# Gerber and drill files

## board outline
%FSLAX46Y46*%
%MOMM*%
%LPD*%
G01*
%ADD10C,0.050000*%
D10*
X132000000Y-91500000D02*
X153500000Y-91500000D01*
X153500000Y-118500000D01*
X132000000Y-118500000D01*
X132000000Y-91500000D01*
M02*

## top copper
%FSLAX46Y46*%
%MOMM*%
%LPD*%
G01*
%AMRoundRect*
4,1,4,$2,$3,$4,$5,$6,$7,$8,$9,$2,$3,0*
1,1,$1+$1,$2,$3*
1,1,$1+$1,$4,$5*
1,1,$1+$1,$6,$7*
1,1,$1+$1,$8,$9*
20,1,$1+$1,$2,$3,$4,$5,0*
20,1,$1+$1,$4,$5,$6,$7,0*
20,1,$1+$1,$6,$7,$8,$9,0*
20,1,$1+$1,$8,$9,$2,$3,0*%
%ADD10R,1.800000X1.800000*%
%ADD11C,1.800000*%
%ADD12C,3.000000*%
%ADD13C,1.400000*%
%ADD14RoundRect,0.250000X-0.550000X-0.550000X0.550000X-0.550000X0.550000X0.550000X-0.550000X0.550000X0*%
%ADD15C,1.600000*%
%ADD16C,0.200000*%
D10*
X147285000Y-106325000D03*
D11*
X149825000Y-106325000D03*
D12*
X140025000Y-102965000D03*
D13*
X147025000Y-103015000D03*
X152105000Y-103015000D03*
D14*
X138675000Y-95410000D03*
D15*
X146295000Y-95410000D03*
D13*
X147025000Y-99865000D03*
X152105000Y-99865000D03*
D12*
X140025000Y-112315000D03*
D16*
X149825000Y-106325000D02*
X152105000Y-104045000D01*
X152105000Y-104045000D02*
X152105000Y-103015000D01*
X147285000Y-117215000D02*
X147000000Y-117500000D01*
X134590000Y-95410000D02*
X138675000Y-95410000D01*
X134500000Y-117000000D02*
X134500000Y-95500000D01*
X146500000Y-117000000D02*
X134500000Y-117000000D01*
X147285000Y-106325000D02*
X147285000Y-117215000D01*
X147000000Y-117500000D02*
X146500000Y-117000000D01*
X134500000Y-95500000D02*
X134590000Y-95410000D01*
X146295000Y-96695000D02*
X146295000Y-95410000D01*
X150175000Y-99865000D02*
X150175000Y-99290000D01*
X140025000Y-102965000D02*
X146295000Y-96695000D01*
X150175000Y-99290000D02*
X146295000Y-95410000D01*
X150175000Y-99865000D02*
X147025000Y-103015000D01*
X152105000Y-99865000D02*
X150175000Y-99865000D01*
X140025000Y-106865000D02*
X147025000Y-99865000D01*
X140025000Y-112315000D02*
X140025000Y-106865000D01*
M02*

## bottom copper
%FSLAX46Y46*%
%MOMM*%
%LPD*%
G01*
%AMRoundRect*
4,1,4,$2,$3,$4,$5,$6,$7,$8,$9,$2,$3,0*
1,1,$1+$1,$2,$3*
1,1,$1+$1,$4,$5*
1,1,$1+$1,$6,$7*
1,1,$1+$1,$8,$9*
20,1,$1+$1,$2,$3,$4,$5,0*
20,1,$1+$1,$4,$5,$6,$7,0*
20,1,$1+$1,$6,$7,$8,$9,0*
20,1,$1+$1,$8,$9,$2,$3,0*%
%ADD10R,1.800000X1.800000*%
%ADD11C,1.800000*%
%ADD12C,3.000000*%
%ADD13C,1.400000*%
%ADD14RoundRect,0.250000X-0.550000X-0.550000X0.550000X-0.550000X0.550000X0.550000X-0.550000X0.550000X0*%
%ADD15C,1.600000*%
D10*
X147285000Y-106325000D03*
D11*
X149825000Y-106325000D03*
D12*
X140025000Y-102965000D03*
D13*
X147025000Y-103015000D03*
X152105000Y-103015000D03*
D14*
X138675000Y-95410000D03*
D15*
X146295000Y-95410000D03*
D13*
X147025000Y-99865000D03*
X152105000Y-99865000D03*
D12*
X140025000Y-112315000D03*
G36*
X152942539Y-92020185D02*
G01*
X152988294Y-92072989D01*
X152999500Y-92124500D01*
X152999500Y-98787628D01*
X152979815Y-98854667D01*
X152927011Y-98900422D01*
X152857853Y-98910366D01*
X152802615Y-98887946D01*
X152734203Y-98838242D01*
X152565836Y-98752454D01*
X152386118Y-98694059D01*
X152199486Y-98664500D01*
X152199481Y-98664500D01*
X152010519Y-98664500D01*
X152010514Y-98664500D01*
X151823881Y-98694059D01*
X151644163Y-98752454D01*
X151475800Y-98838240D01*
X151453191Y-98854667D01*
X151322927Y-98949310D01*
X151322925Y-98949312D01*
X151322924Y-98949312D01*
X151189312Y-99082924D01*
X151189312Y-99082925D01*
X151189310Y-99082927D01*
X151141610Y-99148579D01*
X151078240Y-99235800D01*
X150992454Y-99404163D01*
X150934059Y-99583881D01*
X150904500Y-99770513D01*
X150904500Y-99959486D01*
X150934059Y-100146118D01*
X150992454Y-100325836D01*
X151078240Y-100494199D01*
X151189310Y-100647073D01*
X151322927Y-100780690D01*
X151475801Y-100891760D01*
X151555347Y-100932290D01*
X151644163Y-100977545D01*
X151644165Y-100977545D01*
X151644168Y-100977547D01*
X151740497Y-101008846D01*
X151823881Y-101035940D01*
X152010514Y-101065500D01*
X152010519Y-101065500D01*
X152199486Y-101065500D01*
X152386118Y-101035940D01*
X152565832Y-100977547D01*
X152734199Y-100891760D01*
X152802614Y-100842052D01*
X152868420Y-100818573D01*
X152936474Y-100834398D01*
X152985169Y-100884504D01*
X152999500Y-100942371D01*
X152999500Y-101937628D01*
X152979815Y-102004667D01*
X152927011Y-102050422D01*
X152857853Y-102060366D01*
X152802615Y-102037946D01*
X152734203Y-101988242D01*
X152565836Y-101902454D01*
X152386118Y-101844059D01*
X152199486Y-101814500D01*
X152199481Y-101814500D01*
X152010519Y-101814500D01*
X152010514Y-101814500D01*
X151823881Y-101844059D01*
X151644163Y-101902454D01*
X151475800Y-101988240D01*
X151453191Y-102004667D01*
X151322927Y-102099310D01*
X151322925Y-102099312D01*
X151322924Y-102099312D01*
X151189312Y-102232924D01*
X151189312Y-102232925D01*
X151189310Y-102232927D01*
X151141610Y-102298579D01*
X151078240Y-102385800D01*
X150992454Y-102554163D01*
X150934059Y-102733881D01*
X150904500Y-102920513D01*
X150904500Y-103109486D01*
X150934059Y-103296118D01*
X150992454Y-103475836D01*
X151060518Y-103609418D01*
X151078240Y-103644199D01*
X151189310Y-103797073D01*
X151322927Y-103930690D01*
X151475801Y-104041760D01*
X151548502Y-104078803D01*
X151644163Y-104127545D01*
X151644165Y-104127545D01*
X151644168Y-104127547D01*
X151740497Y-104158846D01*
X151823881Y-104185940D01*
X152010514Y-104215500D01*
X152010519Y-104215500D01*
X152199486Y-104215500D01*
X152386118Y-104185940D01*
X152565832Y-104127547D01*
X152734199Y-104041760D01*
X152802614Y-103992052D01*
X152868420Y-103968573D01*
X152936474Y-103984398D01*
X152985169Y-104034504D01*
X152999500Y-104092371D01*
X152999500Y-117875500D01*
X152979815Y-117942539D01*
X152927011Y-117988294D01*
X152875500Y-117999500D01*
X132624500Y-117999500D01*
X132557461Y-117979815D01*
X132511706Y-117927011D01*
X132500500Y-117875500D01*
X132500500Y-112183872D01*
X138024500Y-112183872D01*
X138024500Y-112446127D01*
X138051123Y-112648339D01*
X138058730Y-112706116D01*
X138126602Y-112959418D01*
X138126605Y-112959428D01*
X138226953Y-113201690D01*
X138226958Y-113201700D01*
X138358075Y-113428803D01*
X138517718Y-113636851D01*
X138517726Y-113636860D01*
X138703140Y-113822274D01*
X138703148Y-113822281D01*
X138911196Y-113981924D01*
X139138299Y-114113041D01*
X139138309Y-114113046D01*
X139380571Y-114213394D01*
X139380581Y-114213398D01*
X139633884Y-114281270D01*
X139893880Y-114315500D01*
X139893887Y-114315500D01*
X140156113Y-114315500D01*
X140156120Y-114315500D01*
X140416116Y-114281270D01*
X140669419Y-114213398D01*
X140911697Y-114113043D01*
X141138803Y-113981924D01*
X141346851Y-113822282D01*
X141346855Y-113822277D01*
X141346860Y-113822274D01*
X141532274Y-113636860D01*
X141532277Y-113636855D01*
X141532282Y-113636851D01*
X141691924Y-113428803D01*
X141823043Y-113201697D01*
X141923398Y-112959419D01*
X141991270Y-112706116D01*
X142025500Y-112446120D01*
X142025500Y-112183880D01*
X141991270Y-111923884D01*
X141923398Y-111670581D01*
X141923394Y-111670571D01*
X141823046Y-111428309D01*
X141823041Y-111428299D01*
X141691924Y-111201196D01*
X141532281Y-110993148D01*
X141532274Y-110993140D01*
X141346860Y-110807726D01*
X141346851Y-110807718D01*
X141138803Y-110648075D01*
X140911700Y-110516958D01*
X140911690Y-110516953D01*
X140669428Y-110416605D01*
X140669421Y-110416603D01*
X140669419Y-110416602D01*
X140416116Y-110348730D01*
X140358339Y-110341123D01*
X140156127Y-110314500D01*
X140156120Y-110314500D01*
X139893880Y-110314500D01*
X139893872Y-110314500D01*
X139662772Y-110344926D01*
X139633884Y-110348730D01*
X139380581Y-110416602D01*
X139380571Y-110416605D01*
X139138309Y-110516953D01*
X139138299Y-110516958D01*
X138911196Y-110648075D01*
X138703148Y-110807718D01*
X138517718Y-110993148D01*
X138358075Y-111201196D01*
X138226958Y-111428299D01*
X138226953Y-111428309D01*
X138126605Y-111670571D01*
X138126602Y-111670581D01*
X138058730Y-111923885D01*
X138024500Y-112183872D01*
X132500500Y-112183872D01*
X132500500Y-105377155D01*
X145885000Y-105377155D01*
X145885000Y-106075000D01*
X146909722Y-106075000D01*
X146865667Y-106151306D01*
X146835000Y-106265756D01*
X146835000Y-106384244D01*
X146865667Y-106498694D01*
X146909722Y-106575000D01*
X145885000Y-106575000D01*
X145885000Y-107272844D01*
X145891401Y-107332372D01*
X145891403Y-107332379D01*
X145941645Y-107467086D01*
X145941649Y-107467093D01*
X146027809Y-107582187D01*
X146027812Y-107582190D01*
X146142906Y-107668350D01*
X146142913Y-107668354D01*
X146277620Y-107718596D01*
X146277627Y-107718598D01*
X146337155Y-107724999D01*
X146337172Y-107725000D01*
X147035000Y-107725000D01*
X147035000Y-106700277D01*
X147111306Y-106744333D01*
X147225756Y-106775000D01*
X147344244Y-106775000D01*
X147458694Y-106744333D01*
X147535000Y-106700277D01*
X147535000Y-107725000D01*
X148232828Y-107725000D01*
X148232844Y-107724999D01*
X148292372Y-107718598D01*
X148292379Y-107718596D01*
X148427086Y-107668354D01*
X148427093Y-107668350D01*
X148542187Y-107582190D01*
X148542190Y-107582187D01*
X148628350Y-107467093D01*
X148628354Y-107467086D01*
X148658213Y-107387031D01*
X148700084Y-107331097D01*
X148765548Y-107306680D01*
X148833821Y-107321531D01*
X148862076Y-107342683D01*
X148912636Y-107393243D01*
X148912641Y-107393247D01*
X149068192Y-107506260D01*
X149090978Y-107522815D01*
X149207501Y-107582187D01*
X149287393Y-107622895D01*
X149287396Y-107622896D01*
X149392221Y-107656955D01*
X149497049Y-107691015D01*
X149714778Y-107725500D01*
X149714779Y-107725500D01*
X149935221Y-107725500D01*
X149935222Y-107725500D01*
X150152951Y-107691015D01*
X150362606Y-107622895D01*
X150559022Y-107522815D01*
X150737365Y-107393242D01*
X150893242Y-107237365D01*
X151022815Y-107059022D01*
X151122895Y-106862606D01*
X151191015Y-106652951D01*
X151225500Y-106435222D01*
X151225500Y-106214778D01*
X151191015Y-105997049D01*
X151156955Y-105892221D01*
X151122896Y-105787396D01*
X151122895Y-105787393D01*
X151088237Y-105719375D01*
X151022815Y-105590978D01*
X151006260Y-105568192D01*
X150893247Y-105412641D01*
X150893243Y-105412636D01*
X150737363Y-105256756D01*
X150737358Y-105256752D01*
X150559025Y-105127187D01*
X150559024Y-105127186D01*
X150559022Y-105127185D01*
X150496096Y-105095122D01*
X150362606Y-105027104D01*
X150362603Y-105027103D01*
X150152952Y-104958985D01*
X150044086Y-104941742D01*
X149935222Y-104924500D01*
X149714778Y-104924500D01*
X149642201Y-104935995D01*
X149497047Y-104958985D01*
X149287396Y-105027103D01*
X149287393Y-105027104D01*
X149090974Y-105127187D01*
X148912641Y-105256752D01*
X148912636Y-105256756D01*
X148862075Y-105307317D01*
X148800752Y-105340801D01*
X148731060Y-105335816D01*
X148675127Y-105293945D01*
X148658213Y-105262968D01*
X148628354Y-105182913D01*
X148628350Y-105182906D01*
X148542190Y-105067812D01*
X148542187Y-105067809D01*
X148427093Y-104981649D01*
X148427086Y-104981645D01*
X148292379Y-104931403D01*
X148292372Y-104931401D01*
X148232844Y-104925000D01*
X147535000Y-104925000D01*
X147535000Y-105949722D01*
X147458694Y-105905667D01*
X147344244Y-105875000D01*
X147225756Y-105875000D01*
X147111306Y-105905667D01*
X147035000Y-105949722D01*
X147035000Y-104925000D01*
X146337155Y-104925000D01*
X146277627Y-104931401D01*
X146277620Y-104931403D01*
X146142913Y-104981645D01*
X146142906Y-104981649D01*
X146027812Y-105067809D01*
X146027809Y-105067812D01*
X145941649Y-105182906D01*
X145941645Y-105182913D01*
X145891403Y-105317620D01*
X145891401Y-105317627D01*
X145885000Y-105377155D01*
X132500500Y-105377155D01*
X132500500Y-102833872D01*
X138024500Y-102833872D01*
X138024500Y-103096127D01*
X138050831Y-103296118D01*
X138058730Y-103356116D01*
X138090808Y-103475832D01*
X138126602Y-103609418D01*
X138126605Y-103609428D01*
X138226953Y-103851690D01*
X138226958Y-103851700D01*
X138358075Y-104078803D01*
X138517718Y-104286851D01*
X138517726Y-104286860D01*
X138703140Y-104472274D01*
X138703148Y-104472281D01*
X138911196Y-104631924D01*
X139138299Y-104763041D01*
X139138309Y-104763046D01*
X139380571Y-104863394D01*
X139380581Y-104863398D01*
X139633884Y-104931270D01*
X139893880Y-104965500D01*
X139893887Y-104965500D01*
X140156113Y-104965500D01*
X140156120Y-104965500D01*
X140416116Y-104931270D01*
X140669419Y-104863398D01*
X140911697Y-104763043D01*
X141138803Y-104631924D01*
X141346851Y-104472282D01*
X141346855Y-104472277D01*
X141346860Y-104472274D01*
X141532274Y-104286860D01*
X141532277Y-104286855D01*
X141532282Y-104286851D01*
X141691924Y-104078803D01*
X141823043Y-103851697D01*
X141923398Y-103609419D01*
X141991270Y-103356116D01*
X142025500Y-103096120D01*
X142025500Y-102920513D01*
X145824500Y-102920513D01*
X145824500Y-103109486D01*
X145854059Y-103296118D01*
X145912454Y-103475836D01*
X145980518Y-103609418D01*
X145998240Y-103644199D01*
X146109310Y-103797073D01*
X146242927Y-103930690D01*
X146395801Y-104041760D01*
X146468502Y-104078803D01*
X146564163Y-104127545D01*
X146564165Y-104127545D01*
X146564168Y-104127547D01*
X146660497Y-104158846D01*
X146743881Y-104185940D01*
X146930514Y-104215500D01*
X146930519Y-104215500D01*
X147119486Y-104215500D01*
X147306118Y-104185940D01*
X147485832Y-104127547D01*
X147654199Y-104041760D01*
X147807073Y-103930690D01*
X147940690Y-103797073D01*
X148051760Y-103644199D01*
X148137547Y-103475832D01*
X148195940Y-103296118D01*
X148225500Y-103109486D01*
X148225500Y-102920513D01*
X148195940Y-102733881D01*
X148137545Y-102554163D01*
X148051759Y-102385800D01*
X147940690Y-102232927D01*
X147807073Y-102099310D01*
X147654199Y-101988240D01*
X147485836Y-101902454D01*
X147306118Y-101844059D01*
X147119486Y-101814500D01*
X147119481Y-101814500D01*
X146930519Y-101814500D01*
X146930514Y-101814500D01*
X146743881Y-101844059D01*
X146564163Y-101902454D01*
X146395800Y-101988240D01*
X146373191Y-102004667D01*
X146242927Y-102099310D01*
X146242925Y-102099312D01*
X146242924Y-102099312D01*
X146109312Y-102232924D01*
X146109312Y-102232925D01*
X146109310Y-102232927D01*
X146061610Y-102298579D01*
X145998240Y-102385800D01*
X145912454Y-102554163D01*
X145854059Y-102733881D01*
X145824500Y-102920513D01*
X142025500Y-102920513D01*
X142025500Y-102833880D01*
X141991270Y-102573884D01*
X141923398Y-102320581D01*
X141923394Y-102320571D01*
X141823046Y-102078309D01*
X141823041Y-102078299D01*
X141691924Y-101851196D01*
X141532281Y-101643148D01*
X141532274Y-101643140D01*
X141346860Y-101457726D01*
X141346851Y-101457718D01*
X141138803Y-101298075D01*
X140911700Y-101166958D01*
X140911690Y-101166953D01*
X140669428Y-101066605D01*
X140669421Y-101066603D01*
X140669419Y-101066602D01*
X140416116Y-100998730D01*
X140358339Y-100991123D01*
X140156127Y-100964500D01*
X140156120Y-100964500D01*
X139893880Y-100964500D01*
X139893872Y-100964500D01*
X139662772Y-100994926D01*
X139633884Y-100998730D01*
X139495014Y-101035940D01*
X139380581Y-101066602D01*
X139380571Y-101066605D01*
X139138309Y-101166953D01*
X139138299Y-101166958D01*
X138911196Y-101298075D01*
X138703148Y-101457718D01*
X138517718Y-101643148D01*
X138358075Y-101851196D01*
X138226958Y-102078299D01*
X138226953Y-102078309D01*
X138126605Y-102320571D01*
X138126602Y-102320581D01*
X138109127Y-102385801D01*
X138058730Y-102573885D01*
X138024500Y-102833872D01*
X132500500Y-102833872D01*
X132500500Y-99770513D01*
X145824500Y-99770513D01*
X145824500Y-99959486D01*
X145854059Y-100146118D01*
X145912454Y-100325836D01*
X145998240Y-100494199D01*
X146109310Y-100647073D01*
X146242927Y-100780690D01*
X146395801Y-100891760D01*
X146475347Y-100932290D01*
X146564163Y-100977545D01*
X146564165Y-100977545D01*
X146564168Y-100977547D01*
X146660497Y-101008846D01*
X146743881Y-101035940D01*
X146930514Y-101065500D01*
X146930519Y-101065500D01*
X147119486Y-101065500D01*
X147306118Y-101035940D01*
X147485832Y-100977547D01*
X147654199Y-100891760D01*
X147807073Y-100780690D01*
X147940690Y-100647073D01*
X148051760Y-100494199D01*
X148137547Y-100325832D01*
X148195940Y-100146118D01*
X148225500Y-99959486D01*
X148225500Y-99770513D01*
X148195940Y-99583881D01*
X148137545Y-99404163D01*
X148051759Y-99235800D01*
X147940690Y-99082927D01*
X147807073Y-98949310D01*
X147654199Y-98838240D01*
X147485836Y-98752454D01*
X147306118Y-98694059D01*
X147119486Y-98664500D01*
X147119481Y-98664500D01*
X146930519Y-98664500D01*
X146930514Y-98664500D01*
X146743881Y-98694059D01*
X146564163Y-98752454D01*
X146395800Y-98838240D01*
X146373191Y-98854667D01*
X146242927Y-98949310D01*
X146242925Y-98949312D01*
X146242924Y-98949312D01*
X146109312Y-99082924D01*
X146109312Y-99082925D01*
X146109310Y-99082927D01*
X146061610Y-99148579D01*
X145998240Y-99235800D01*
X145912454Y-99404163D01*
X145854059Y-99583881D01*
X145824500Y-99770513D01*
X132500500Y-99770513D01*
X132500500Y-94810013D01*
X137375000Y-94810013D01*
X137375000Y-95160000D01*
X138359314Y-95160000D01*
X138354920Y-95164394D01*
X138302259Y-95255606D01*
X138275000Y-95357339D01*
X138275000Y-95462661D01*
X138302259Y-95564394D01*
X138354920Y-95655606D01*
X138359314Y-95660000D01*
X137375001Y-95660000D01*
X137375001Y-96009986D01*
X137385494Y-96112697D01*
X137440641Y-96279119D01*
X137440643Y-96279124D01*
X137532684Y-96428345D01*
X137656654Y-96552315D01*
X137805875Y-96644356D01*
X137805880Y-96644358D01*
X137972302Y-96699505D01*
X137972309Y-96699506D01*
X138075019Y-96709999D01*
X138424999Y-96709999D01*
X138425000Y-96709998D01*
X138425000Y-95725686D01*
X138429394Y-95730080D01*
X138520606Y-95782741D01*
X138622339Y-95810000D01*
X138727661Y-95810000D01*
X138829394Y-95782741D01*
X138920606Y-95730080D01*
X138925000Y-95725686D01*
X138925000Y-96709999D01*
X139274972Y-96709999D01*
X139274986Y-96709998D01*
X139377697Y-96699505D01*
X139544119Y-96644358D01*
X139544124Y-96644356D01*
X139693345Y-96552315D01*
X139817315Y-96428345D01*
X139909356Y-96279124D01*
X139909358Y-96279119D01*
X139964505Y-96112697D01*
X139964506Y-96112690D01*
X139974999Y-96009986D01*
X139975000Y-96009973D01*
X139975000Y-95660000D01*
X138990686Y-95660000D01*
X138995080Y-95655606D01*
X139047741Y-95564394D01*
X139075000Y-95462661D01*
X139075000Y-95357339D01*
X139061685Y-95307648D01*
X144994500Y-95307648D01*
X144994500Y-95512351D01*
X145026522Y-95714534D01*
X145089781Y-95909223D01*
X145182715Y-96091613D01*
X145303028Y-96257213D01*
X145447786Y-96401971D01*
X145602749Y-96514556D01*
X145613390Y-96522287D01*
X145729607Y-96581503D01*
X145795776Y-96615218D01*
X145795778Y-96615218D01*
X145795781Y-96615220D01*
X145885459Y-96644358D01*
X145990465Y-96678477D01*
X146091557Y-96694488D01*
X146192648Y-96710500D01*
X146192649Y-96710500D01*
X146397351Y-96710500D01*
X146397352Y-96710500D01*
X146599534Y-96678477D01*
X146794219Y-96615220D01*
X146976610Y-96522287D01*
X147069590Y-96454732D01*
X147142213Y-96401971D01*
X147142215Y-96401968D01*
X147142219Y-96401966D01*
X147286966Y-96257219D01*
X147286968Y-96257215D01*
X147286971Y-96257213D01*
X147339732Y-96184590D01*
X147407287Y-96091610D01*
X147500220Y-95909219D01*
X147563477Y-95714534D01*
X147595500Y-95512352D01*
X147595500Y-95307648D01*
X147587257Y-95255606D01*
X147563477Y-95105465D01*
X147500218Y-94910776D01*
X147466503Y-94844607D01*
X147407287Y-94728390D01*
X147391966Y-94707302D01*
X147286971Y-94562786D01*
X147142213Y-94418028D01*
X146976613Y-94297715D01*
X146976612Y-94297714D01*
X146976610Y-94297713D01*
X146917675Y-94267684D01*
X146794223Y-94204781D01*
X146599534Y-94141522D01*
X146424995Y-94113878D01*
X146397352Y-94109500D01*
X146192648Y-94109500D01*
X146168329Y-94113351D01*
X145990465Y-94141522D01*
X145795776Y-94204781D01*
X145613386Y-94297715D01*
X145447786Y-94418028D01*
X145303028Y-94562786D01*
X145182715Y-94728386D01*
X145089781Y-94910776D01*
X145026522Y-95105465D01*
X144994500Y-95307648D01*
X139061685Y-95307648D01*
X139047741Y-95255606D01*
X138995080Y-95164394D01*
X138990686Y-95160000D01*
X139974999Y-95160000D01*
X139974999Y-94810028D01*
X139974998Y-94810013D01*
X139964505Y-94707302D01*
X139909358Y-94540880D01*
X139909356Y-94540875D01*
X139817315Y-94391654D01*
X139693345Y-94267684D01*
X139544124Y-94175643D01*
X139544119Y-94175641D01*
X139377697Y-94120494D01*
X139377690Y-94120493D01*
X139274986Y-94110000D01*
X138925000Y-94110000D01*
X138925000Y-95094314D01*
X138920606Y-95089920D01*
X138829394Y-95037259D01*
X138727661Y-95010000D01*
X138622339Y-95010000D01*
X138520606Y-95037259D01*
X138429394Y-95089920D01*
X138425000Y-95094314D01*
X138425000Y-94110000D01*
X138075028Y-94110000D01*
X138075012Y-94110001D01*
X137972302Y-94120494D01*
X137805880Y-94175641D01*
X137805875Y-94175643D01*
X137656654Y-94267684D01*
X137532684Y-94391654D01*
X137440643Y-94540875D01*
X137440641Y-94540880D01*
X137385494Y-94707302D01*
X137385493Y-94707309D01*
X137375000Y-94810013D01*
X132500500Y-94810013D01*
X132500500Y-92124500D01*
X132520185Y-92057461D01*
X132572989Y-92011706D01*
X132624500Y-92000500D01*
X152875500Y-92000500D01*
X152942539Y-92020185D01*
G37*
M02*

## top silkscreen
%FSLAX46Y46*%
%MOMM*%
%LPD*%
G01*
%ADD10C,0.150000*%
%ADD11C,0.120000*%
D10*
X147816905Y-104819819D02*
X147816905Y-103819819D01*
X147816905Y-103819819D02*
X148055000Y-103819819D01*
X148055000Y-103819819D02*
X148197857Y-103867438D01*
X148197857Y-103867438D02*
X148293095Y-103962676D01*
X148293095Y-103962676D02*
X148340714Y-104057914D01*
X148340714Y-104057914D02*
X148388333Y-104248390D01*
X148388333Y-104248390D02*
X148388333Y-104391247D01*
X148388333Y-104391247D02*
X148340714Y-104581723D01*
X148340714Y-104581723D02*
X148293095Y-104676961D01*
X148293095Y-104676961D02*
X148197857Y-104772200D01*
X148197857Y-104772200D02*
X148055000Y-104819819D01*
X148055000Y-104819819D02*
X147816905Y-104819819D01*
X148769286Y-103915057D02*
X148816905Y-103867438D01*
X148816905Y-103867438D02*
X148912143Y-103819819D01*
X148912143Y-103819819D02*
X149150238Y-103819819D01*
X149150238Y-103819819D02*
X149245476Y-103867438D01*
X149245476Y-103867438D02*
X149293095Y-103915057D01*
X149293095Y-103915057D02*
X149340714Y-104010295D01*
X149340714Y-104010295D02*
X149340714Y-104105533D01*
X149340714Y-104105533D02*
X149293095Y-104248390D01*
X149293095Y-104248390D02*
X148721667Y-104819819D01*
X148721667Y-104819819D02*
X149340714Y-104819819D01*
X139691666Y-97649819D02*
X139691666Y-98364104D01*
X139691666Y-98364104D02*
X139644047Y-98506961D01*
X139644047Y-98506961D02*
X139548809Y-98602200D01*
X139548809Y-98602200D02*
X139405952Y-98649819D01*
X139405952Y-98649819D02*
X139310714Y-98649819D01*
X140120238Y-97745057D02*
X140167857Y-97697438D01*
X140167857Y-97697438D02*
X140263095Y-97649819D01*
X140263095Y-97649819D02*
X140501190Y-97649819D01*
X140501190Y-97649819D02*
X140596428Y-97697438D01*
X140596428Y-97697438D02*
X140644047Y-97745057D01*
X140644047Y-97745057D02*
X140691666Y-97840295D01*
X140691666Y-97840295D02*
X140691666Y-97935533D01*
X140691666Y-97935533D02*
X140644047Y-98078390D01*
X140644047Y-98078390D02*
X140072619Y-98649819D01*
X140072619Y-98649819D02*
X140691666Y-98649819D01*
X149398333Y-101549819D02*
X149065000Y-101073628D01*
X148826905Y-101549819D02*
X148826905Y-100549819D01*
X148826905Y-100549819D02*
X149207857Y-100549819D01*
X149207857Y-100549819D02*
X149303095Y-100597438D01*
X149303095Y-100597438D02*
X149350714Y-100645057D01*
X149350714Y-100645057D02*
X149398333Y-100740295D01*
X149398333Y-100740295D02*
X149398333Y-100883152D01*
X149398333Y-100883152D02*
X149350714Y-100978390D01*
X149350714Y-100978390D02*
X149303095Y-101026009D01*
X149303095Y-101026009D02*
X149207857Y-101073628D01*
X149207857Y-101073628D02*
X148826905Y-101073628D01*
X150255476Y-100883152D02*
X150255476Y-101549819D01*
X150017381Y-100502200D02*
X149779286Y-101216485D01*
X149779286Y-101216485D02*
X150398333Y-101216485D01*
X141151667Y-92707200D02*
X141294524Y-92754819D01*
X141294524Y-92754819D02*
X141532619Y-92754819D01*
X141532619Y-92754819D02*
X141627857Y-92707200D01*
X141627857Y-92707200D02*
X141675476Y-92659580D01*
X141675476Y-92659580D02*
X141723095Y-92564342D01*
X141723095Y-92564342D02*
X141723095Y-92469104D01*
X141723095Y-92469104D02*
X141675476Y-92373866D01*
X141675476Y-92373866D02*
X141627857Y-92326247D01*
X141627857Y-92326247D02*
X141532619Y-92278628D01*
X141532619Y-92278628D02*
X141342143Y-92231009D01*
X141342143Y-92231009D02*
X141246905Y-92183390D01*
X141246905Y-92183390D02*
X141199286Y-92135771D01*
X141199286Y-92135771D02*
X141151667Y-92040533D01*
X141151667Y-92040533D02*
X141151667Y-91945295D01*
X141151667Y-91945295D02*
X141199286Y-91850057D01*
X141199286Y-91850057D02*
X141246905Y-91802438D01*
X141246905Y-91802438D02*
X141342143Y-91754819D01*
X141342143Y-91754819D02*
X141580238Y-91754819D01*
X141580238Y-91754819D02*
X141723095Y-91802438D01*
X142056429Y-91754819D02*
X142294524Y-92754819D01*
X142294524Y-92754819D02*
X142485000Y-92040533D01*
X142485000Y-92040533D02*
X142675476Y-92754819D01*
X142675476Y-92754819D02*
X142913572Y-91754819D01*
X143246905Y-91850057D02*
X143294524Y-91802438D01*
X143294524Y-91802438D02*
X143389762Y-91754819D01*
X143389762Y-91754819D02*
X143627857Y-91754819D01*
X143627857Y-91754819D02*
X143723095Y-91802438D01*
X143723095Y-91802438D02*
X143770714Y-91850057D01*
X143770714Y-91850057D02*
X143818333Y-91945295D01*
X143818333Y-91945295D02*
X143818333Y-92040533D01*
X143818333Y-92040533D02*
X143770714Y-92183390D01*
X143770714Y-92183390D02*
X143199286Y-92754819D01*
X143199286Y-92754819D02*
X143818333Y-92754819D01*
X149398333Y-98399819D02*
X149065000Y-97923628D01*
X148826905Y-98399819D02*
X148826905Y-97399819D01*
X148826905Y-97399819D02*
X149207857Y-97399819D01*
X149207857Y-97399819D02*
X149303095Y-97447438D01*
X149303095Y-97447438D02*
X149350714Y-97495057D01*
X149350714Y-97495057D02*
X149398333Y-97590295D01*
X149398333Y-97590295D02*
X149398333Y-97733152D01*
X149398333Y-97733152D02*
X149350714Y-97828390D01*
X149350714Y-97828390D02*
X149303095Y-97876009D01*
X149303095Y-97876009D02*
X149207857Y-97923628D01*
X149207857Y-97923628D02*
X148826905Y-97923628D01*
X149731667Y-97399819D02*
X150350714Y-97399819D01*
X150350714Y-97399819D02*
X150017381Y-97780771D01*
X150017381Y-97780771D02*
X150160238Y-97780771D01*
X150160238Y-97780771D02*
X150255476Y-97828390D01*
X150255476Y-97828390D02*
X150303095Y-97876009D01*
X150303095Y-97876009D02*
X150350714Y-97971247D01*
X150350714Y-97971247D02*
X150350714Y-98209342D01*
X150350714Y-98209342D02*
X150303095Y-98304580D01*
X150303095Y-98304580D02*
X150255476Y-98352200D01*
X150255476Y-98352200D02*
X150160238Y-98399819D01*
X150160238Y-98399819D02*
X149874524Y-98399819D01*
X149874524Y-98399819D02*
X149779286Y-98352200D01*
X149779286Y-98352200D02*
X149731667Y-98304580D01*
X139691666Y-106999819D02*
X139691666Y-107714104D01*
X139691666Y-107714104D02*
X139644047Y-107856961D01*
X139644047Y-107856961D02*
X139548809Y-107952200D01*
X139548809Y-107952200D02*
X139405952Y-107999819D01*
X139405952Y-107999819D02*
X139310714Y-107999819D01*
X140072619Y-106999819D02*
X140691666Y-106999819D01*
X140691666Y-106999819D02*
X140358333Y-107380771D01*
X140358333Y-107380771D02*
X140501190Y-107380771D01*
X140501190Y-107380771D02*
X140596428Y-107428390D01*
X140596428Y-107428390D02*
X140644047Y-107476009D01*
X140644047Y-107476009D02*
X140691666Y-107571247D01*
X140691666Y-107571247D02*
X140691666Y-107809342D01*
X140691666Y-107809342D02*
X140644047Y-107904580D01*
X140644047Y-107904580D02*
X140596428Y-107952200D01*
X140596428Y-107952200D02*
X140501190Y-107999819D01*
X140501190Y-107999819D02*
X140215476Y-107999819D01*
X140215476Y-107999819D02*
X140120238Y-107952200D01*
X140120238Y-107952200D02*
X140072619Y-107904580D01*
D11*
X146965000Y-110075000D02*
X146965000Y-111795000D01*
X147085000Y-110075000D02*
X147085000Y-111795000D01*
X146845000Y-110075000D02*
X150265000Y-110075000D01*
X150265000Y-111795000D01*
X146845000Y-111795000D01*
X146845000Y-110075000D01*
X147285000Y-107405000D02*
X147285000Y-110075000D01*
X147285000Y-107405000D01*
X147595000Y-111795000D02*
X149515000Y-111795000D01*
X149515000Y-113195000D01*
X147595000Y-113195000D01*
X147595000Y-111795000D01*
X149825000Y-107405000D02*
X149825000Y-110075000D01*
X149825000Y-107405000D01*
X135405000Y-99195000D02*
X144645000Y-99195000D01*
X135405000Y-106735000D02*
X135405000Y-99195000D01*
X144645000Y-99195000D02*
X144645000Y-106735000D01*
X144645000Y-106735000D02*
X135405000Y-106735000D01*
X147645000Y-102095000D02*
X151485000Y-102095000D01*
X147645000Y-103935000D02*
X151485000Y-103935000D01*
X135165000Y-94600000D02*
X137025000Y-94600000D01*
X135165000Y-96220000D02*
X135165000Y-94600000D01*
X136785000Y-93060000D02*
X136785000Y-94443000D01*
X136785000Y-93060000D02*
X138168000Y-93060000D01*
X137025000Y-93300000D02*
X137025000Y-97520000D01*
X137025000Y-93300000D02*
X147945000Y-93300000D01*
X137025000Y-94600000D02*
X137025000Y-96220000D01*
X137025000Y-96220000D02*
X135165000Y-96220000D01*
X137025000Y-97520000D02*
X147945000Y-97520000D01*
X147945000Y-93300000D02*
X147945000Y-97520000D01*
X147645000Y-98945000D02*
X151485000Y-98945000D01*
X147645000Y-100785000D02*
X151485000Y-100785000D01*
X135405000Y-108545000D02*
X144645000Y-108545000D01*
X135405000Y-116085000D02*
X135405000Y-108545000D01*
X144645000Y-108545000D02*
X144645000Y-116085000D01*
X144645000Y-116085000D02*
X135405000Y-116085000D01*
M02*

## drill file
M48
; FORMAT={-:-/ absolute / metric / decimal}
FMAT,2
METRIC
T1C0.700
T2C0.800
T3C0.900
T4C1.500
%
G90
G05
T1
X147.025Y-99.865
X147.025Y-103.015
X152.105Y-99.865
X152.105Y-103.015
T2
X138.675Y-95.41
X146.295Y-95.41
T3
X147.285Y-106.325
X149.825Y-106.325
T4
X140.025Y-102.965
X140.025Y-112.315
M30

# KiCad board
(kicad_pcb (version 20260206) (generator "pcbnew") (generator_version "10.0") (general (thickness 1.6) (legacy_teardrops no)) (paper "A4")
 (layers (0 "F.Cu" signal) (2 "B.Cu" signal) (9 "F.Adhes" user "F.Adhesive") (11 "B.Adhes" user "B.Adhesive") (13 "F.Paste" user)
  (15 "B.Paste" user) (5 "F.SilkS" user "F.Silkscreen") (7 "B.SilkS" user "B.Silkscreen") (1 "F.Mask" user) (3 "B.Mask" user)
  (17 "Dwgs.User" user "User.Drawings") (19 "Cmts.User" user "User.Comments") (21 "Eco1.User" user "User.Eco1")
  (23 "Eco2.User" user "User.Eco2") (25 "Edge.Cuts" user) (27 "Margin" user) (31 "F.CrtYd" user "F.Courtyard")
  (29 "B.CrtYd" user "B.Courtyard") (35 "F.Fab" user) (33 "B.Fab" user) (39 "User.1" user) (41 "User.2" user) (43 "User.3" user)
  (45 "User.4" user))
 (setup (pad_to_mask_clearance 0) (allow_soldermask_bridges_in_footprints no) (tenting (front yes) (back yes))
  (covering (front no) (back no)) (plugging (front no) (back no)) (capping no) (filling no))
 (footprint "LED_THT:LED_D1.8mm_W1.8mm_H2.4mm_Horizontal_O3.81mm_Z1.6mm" (layer "F.Cu") (at 147.285 106.325)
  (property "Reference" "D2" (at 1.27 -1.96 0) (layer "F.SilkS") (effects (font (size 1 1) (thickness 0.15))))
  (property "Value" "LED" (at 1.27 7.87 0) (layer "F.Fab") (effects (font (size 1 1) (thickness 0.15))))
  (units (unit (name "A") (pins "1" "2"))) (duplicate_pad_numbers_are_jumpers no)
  (fp_line (start -0.32 3.75) (end -0.32 5.47) (stroke (width 0.12) (type solid)) (layer "F.SilkS"))
  (fp_line (start -0.2 3.75) (end -0.2 5.47) (stroke (width 0.12) (type solid)) (layer "F.SilkS"))
  (fp_rect (start -0.44 3.75) (end 2.98 5.47) (stroke (width 0.12) (type solid)) (fill no) (layer "F.SilkS"))
  (fp_rect (start 0 1.08) (end 0 3.75) (stroke (width 0.12) (type solid)) (fill no) (layer "F.SilkS"))
  (fp_rect (start 0.31 5.47) (end 2.23 6.87) (stroke (width 0.12) (type solid)) (fill no) (layer "F.SilkS"))
  (fp_rect (start 2.54 1.08) (end 2.54 3.75) (stroke (width 0.12) (type solid)) (fill no) (layer "F.SilkS"))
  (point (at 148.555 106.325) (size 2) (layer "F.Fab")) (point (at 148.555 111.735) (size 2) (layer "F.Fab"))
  (pad "1" thru_hole rect (at 0 0) (size 1.8 1.8) (drill 0.9) (layers "*.Cu" "*.Mask") (remove_unused_layers no) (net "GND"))
  (pad "2" thru_hole circle (at 2.54 0) (size 1.8 1.8) (drill 0.9) (layers "*.Cu" "*.Mask") (remove_unused_layers no) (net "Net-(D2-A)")))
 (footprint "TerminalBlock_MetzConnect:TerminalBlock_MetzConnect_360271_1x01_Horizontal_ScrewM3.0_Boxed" (layer "F.Cu") (at 140.025 102.965)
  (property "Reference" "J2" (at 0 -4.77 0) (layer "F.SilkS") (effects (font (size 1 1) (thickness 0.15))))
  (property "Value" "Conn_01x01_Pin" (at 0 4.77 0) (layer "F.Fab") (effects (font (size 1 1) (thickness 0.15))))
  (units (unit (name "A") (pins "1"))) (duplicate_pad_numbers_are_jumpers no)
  (fp_line (start -4.62 -3.77) (end 4.62 -3.77) (stroke (width 0.12) (type solid)) (layer "F.SilkS"))
  (fp_line (start -4.62 3.77) (end -4.62 -3.77) (stroke (width 0.12) (type solid)) (layer "F.SilkS"))
  (fp_line (start 4.62 -3.77) (end 4.62 3.77) (stroke (width 0.12) (type solid)) (layer "F.SilkS"))
  (fp_line (start 4.62 3.77) (end -4.62 3.77) (stroke (width 0.12) (type solid)) (layer "F.SilkS"))
  (pad "1" thru_hole circle (at 0 0) (size 3 3) (drill 1.5) (layers "*.Cu" "*.Mask") (remove_unused_layers no) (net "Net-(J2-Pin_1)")))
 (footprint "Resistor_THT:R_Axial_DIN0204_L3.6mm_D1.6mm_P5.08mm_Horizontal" (layer "F.Cu") (at 147.025 103.015)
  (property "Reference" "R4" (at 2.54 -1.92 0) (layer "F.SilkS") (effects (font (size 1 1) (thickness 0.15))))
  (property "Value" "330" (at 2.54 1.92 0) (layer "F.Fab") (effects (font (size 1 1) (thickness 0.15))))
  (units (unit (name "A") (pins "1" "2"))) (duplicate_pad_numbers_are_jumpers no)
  (fp_line (start 0.62 -0.92) (end 4.46 -0.92) (stroke (width 0.12) (type solid)) (layer "F.SilkS"))
  (fp_line (start 0.62 0.92) (end 4.46 0.92) (stroke (width 0.12) (type solid)) (layer "F.SilkS"))
  (pad "1" thru_hole circle (at 0 0) (size 1.4 1.4) (drill 0.7) (layers "*.Cu" "*.Mask") (remove_unused_layers no) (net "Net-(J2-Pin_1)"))
  (pad "2" thru_hole circle (at 5.08 0) (size 1.4 1.4) (drill 0.7) (layers "*.Cu" "*.Mask") (remove_unused_layers no) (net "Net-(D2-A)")))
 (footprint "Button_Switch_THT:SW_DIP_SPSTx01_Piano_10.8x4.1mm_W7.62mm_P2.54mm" (layer "F.Cu") (at 138.675 95.41)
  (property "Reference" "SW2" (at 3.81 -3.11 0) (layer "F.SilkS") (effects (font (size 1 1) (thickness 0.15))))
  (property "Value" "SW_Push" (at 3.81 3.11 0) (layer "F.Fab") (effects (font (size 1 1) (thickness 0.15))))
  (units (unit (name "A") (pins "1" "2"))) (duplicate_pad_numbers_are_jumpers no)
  (fp_line (start -3.51 -0.81) (end -1.65 -0.81) (stroke (width 0.12) (type solid)) (layer "F.SilkS"))
  (fp_line (start -3.51 0.81) (end -3.51 -0.81) (stroke (width 0.12) (type solid)) (layer "F.SilkS"))
  (fp_line (start -1.89 -2.35) (end -1.89 -0.967) (stroke (width 0.12) (type solid)) (layer "F.SilkS"))
  (fp_line (start -1.89 -2.35) (end -0.507 -2.35) (stroke (width 0.12) (type solid)) (layer "F.SilkS"))
  (fp_line (start -1.65 -2.11) (end -1.65 2.11) (stroke (width 0.12) (type solid)) (layer "F.SilkS"))
  (fp_line (start -1.65 -2.11) (end 9.27 -2.11) (stroke (width 0.12) (type solid)) (layer "F.SilkS"))
  (fp_line (start -1.65 -0.81) (end -1.65 0.81) (stroke (width 0.12) (type solid)) (layer "F.SilkS"))
  (fp_line (start -1.65 0.81) (end -3.51 0.81) (stroke (width 0.12) (type solid)) (layer "F.SilkS"))
  (fp_line (start -1.65 2.11) (end 9.27 2.11) (stroke (width 0.12) (type solid)) (layer "F.SilkS"))
  (fp_line (start 9.27 -2.11) (end 9.27 2.11) (stroke (width 0.12) (type solid)) (layer "F.SilkS"))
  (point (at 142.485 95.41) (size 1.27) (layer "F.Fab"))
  (pad "1" thru_hole roundrect (at 0 0) (size 1.6 1.6) (drill 0.8) (layers "*.Cu" "*.Mask") (remove_unused_layers no)
   (roundrect_rratio 0.15625) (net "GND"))
  (pad "2" thru_hole circle (at 7.62 0) (size 1.6 1.6) (drill 0.8) (layers "*.Cu" "*.Mask") (remove_unused_layers no) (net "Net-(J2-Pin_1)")))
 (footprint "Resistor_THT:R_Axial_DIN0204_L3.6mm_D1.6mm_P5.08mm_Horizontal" (layer "F.Cu") (at 147.025 99.865)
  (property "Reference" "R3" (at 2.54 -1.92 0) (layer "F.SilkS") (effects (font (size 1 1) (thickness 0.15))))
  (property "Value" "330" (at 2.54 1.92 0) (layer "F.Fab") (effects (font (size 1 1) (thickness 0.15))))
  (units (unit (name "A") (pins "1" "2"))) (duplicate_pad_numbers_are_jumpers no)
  (fp_line (start 0.62 -0.92) (end 4.46 -0.92) (stroke (width 0.12) (type solid)) (layer "F.SilkS"))
  (fp_line (start 0.62 0.92) (end 4.46 0.92) (stroke (width 0.12) (type solid)) (layer "F.SilkS"))
  (pad "1" thru_hole circle (at 0 0) (size 1.4 1.4) (drill 0.7) (layers "*.Cu" "*.Mask") (remove_unused_layers no) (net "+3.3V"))
  (pad "2" thru_hole circle (at 5.08 0) (size 1.4 1.4) (drill 0.7) (layers "*.Cu" "*.Mask") (remove_unused_layers no) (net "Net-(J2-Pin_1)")))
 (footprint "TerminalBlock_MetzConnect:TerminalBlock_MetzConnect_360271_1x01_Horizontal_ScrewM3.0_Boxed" (layer "F.Cu") (at 140.025 112.315)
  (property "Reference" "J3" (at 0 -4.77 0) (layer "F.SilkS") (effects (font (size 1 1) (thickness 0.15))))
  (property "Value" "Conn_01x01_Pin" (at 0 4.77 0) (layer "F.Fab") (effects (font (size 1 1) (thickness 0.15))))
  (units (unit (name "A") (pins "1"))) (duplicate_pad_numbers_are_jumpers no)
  (fp_line (start -4.62 -3.77) (end 4.62 -3.77) (stroke (width 0.12) (type solid)) (layer "F.SilkS"))
  (fp_line (start -4.62 3.77) (end -4.62 -3.77) (stroke (width 0.12) (type solid)) (layer "F.SilkS"))
  (fp_line (start 4.62 -3.77) (end 4.62 3.77) (stroke (width 0.12) (type solid)) (layer "F.SilkS"))
  (fp_line (start 4.62 3.77) (end -4.62 3.77) (stroke (width 0.12) (type solid)) (layer "F.SilkS"))
  (pad "1" thru_hole circle (at 0 0) (size 3 3) (drill 1.5) (layers "*.Cu" "*.Mask") (remove_unused_layers no) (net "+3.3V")))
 (gr_rect (start 132 91.5) (end 153.5 118.5) (stroke (width 0.05) (type default)) (fill no) (layer "Edge.Cuts"))
 (segment (start 149.825 106.325) (end 152.105 104.045) (width 0.2) (layer "F.Cu") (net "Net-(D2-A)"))
 (segment (start 152.105 104.045) (end 152.105 103.015) (width 0.2) (layer "F.Cu") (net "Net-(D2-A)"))
 (segment (start 147.285 117.215) (end 147 117.5) (width 0.2) (layer "F.Cu") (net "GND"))
 (segment (start 134.59 95.41) (end 138.675 95.41) (width 0.2) (layer "F.Cu") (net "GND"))
 (segment (start 134.5 117) (end 134.5 95.5) (width 0.2) (layer "F.Cu") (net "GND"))
 (segment (start 146.5 117) (end 134.5 117) (width 0.2) (layer "F.Cu") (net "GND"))
 (segment (start 147.285 106.325) (end 147.285 117.215) (width 0.2) (layer "F.Cu") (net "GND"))
 (segment (start 147 117.5) (end 146.5 117) (width 0.2) (layer "F.Cu") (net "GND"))
 (segment (start 134.5 95.5) (end 134.59 95.41) (width 0.2) (layer "F.Cu") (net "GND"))
 (segment (start 146.295 96.695) (end 146.295 95.41) (width 0.2) (layer "F.Cu") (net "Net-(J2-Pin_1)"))
 (segment (start 150.175 99.865) (end 150.175 99.29) (width 0.2) (layer "F.Cu") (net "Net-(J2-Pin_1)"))
 (segment (start 140.025 102.965) (end 146.295 96.695) (width 0.2) (layer "F.Cu") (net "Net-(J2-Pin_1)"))
 (segment (start 150.175 99.29) (end 146.295 95.41) (width 0.2) (layer "F.Cu") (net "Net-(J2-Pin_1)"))
 (segment (start 150.175 99.865) (end 147.025 103.015) (width 0.2) (layer "F.Cu") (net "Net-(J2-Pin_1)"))
 (segment (start 152.105 99.865) (end 150.175 99.865) (width 0.2) (layer "F.Cu") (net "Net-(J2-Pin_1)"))
 (segment (start 140.025 106.865) (end 147.025 99.865) (width 0.2) (layer "F.Cu") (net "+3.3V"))
 (segment (start 140.025 112.315) (end 140.025 106.865) (width 0.2) (layer "F.Cu") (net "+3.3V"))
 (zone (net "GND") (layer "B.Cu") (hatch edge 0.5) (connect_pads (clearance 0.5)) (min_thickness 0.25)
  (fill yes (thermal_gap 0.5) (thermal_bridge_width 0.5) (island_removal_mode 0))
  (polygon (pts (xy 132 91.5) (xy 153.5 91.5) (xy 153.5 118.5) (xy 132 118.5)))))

